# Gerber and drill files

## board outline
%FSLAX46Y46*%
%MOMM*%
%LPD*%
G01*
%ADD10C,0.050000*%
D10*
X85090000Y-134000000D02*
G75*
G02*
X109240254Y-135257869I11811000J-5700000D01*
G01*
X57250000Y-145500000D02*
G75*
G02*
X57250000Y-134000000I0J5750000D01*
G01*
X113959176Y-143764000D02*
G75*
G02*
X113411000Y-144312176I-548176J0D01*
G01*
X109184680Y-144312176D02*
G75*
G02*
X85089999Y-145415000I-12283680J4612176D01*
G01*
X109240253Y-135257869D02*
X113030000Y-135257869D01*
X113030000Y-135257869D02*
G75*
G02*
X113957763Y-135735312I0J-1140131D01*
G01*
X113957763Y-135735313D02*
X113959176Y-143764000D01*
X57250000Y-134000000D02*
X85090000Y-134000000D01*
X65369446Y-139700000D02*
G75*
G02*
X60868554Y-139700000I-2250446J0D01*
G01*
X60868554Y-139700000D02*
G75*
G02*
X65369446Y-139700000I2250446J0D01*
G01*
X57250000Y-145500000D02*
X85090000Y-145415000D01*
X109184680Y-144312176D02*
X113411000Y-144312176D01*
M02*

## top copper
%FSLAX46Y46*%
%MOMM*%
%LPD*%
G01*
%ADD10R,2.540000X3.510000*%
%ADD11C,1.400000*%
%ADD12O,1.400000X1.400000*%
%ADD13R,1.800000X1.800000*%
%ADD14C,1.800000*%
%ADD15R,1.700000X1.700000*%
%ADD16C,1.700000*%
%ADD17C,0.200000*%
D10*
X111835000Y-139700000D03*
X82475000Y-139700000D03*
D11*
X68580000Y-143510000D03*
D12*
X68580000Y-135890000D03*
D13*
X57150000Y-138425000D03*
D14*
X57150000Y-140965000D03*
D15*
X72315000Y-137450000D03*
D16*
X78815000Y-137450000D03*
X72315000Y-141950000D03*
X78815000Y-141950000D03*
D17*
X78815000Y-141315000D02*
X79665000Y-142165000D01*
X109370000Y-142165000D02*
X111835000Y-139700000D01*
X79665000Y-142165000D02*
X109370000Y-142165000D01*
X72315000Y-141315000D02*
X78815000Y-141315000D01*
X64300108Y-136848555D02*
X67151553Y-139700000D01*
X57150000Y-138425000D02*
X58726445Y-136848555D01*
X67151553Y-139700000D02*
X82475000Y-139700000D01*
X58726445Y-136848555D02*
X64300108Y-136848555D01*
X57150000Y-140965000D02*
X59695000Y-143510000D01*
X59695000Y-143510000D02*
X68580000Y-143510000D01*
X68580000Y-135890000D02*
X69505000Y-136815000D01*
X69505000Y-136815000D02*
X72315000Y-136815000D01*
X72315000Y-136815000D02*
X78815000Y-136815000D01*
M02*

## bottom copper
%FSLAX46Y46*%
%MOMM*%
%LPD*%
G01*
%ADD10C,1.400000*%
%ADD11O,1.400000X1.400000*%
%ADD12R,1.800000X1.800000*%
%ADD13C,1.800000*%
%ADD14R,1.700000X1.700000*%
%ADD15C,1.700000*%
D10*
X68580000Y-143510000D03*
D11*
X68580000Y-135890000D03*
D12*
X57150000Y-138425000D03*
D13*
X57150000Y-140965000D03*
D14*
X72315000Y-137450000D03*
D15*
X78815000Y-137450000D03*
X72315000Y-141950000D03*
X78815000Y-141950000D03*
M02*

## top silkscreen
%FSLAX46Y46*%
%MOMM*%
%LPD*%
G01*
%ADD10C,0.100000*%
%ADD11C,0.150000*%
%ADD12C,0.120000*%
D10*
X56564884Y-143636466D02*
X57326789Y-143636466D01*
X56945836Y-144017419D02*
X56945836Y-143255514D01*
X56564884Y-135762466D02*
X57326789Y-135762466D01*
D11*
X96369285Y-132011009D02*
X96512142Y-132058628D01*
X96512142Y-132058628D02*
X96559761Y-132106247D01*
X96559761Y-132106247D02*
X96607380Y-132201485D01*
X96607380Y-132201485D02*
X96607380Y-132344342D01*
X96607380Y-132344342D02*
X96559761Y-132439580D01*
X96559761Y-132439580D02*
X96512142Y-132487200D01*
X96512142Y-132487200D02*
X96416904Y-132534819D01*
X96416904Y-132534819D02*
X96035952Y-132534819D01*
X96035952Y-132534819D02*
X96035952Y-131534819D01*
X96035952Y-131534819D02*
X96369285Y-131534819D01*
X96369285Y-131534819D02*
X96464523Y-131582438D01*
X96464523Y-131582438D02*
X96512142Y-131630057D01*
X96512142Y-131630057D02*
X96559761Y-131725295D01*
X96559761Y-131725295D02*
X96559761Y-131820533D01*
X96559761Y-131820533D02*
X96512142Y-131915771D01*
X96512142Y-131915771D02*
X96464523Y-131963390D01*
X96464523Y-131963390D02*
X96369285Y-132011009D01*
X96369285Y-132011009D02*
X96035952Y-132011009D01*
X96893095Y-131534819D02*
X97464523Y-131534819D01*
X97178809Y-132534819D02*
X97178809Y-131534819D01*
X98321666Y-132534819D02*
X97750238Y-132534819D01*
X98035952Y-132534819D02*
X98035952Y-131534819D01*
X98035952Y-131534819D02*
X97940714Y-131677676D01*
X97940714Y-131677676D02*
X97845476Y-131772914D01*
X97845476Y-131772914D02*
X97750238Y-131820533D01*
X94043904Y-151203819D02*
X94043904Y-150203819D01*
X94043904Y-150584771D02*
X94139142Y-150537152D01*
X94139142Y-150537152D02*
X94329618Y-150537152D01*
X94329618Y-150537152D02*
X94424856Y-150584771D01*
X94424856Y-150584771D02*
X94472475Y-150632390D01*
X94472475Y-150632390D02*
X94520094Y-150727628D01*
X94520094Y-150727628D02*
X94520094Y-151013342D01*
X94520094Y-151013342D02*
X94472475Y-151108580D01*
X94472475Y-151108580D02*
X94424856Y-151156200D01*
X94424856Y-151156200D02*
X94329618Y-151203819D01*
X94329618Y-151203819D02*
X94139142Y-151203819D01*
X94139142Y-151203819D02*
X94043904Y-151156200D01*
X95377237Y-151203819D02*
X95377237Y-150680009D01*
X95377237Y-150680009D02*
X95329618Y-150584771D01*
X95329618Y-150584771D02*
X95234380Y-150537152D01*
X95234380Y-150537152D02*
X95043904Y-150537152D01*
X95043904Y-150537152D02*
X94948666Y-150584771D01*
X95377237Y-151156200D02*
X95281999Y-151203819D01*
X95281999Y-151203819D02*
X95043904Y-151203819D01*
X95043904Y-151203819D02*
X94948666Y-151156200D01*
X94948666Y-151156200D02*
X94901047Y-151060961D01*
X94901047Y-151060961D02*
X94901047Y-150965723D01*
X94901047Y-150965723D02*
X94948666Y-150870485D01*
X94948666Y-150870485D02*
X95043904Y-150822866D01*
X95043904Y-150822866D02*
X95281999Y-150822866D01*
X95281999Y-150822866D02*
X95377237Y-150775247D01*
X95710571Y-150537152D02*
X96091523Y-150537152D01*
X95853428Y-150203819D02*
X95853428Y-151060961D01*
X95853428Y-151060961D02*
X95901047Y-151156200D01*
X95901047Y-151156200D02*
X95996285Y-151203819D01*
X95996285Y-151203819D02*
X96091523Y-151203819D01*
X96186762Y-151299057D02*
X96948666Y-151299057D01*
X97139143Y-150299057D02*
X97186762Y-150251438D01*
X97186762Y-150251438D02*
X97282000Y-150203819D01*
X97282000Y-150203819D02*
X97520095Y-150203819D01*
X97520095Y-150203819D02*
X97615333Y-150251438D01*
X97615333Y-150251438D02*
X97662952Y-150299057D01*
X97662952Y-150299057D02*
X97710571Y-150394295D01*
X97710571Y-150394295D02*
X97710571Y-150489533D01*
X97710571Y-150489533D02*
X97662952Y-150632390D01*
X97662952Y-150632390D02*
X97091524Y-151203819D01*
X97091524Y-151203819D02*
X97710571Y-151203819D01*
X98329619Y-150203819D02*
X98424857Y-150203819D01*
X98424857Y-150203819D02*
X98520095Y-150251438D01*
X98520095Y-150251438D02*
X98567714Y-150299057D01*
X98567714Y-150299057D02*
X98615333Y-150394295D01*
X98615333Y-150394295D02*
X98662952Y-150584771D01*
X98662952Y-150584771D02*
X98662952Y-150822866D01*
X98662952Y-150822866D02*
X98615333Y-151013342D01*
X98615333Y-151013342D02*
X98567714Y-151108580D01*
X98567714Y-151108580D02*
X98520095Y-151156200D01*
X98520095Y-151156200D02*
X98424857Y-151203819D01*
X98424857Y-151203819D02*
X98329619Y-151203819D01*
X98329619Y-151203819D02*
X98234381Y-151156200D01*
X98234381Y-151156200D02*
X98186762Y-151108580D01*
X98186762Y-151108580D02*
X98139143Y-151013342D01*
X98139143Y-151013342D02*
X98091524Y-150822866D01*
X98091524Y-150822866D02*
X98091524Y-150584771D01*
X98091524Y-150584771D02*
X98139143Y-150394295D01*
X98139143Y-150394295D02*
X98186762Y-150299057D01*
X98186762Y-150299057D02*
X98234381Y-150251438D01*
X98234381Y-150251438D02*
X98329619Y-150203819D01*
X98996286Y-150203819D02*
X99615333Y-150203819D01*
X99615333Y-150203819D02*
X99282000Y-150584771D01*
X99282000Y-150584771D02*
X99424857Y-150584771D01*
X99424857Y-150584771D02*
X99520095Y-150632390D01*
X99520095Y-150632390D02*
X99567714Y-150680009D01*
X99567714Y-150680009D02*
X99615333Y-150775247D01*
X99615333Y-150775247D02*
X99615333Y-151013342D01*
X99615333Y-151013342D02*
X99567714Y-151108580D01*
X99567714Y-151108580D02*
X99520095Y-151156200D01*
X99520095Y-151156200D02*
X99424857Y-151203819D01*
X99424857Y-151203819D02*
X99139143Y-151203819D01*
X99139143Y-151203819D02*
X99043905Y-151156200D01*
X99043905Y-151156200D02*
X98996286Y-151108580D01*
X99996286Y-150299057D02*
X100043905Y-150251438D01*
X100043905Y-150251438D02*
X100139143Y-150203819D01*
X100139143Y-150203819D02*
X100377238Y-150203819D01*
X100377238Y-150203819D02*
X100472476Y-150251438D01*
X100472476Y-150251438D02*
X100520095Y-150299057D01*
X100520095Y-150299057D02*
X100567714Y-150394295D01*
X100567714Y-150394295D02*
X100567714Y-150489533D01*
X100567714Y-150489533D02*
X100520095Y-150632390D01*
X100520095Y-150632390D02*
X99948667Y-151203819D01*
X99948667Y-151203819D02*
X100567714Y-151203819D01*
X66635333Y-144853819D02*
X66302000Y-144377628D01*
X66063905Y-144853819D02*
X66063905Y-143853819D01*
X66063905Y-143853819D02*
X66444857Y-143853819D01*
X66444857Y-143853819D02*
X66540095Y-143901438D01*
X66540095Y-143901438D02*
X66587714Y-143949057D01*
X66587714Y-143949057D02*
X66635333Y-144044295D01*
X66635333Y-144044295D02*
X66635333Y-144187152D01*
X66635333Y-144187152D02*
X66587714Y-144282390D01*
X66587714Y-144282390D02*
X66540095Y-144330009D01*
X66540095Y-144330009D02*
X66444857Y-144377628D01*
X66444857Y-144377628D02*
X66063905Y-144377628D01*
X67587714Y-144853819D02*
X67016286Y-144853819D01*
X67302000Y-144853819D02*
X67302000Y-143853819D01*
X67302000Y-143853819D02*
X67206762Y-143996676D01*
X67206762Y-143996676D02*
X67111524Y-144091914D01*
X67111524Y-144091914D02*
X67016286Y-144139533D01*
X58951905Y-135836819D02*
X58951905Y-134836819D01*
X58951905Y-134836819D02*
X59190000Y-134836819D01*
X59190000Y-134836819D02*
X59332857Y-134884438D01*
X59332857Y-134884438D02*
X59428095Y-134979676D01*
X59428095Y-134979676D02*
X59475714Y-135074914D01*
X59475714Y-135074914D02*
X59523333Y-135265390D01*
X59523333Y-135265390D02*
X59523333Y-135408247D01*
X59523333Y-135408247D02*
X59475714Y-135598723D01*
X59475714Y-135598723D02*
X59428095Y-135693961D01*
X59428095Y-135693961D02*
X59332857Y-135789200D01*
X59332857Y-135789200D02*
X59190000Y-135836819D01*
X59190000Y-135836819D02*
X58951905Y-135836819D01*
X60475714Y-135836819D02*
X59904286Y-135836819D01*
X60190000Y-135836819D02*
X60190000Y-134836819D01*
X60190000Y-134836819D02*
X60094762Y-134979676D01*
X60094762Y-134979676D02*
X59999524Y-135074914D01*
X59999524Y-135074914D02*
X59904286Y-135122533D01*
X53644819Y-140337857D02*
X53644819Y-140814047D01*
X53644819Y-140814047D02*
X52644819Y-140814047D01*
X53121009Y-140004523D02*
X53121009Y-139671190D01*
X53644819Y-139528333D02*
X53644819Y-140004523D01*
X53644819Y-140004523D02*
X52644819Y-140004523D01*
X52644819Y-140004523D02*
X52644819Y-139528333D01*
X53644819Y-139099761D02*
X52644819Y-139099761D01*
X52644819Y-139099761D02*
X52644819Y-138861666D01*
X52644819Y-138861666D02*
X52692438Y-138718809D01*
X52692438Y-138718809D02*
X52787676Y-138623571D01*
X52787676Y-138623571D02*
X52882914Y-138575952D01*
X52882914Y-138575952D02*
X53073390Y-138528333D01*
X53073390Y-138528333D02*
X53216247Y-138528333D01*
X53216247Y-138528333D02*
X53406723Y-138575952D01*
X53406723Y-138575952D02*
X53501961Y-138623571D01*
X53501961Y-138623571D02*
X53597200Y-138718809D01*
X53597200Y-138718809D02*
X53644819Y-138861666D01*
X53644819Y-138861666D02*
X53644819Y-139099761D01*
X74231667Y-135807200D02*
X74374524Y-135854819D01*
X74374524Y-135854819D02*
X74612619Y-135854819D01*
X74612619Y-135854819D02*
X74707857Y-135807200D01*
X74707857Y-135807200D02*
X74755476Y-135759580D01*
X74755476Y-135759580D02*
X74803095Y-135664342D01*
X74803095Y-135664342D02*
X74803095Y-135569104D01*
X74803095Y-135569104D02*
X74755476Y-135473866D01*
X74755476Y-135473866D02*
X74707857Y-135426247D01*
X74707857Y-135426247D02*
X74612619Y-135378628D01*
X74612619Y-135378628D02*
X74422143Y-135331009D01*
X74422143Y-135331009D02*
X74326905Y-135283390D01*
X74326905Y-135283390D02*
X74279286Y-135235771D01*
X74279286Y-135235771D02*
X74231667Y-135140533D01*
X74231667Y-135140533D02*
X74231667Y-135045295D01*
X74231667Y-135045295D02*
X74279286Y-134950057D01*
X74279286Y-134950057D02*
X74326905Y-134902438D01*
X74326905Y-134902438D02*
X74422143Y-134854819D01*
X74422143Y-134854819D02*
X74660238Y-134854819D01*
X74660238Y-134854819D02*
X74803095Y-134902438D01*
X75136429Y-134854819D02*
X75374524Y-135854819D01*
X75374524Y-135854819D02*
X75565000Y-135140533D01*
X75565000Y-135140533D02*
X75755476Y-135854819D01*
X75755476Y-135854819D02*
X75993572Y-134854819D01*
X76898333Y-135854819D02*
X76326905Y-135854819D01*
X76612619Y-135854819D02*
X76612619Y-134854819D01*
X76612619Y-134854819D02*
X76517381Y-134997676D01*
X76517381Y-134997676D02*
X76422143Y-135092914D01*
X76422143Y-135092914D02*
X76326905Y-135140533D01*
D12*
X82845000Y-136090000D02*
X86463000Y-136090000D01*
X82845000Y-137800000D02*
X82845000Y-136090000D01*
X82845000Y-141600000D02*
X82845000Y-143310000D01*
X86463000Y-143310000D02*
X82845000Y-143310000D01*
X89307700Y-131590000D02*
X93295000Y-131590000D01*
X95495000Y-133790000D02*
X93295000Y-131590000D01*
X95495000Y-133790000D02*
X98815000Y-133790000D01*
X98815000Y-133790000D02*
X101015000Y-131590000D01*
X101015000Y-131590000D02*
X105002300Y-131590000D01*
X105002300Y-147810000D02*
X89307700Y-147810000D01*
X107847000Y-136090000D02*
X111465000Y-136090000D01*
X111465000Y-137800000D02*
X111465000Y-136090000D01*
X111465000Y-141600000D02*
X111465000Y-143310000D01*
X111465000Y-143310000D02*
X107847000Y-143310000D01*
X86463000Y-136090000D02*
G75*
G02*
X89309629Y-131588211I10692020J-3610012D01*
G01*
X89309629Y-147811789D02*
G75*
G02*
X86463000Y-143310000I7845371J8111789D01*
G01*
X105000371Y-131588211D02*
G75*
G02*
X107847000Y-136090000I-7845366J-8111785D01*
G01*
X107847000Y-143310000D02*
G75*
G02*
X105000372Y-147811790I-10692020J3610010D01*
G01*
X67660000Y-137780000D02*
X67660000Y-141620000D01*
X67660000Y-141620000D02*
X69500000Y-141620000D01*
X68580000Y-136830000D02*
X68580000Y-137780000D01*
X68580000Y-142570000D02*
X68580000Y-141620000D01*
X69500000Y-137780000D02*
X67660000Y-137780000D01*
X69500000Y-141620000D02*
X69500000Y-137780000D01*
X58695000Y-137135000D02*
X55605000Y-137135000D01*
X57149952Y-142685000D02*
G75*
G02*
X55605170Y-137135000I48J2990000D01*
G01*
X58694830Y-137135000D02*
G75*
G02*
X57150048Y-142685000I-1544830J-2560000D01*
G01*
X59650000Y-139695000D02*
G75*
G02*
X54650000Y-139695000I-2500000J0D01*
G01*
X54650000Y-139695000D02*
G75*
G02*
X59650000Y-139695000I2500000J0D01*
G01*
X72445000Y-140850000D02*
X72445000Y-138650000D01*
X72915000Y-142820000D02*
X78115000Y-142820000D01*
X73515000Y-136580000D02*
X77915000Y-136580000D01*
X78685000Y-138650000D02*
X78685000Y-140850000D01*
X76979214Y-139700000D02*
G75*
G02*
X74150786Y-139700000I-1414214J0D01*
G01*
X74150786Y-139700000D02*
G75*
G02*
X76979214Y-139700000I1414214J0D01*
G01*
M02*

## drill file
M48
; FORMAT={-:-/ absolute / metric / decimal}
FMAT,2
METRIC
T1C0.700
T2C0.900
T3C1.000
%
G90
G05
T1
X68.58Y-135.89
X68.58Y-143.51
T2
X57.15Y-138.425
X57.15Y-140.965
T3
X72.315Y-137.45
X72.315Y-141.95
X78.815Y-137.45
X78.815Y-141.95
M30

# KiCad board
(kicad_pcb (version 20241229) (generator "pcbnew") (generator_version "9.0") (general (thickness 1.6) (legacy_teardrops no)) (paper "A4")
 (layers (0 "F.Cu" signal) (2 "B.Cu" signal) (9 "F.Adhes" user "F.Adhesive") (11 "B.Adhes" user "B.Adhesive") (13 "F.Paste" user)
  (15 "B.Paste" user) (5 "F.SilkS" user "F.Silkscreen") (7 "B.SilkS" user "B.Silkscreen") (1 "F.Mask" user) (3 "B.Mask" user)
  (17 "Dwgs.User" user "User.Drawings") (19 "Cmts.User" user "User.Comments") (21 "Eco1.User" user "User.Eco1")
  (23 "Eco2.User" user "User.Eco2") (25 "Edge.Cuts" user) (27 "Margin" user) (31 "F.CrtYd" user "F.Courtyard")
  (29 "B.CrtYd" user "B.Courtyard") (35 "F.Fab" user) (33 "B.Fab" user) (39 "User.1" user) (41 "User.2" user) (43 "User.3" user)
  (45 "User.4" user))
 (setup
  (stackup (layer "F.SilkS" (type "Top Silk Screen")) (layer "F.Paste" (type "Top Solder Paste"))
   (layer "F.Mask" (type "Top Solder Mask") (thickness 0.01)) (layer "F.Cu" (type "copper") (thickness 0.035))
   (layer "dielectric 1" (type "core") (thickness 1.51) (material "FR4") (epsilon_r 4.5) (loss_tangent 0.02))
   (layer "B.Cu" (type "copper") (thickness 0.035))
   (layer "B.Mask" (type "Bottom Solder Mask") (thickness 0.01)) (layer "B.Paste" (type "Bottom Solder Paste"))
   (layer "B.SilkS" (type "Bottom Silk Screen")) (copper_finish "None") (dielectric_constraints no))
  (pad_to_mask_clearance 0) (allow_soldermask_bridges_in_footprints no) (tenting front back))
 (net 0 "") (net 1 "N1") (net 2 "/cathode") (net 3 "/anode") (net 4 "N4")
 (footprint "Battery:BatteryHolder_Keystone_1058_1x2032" (layer "F.Cu") (at 97.155 139.7 180)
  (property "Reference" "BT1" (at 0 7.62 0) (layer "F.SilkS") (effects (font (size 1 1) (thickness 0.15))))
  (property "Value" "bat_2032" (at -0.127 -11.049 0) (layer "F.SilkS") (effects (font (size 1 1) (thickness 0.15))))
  (fp_line (start 14.31 3.61) (end 10.692 3.61) (stroke (width 0.12) (type solid)) (layer "F.SilkS"))
  (fp_line (start 14.31 1.9) (end 14.31 3.61) (stroke (width 0.12) (type solid)) (layer "F.SilkS"))
  (fp_line (start 14.31 -1.9) (end 14.31 -3.61) (stroke (width 0.12) (type solid)) (layer "F.SilkS"))
  (fp_line (start 10.692 -3.61) (end 14.31 -3.61) (stroke (width 0.12) (type solid)) (layer "F.SilkS"))
  (fp_line (start 7.8473 8.11) (end 3.86 8.11) (stroke (width 0.12) (type solid)) (layer "F.SilkS"))
  (fp_line (start 1.66 5.91) (end 3.86 8.11) (stroke (width 0.12) (type solid)) (layer "F.SilkS"))
  (fp_line (start 1.66 5.91) (end -1.66 5.91) (stroke (width 0.12) (type solid)) (layer "F.SilkS"))
  (fp_line (start -1.66 5.91) (end -3.86 8.11) (stroke (width 0.12) (type solid)) (layer "F.SilkS"))
  (fp_line (start -3.86 8.11) (end -7.8473 8.11) (stroke (width 0.12) (type solid)) (layer "F.SilkS"))
  (fp_line (start -7.8473 -8.11) (end 7.8473 -8.11) (stroke (width 0.12) (type solid)) (layer "F.SilkS"))
  (fp_line (start -10.692 3.61) (end -14.31 3.61) (stroke (width 0.12) (type solid)) (layer "F.SilkS"))
  (fp_line (start -14.31 1.9) (end -14.31 3.61) (stroke (width 0.12) (type solid)) (layer "F.SilkS"))
  (fp_line (start -14.31 -1.9) (end -14.31 -3.61) (stroke (width 0.12) (type solid)) (layer "F.SilkS"))
  (fp_line (start -14.31 -3.61) (end -10.692 -3.61) (stroke (width 0.12) (type solid)) (layer "F.SilkS"))
  (fp_arc (start 10.692 3.61) (mid 9.538084 6.031244) (end 7.845371 8.111789) (stroke (width 0.12) (type solid)) (layer "F.SilkS"))
  (fp_arc (start 7.845371 -8.111789) (mid 9.538085 -6.031244) (end 10.692 -3.61) (stroke (width 0.12) (type solid)) (layer "F.SilkS"))
  (fp_arc (start -7.845371 8.111789) (mid -9.538085 6.031244) (end -10.692 3.61) (stroke (width 0.12) (type solid)) (layer "F.SilkS"))
  (fp_arc (start -10.692 -3.61) (mid -9.538084 -6.031244) (end -7.845371 -8.111789) (stroke (width 0.12) (type solid)) (layer "F.SilkS"))
  (pad "1" smd rect (at -14.68 0 180) (size 2.54 3.51) (layers "F.Cu" "F.Mask" "F.Paste") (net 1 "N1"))
  (pad "2" smd rect (at 14.68 0 180) (size 2.54 3.51) (layers "F.Cu" "F.Mask" "F.Paste") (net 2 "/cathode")))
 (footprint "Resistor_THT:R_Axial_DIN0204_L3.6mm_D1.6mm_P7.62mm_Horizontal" (layer "F.Cu") (at 68.58 143.51 90)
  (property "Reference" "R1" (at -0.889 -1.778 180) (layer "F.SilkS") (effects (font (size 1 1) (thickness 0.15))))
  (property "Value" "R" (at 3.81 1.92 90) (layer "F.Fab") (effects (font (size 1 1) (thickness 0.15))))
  (fp_line (start 5.73 -0.92) (end 1.89 -0.92) (stroke (width 0.12) (type solid)) (layer "F.SilkS"))
  (fp_line (start 1.89 -0.92) (end 1.89 0.92) (stroke (width 0.12) (type solid)) (layer "F.SilkS"))
  (fp_line (start 6.68 0) (end 5.73 0) (stroke (width 0.12) (type solid)) (layer "F.SilkS"))
  (fp_line (start 0.94 0) (end 1.89 0) (stroke (width 0.12) (type solid)) (layer "F.SilkS"))
  (fp_line (start 5.73 0.92) (end 5.73 -0.92) (stroke (width 0.12) (type solid)) (layer "F.SilkS"))
  (fp_line (start 1.89 0.92) (end 5.73 0.92) (stroke (width 0.12) (type solid)) (layer "F.SilkS"))
  (pad "1" thru_hole circle (at 0 0 90) (size 1.4 1.4) (drill 0.7) (layers "*.Cu" "*.Mask") (remove_unused_layers no) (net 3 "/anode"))
  (pad "2" thru_hole oval (at 7.62 0 90) (size 1.4 1.4) (drill 0.7) (layers "*.Cu" "*.Mask") (remove_unused_layers no) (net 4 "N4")))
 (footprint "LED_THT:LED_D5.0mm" (layer "F.Cu") (at 57.15 138.425 -90)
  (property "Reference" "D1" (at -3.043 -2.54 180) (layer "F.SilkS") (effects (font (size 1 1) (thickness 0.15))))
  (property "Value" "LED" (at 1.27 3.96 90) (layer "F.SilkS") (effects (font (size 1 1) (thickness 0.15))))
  (fp_line (start -1.29 -1.545) (end -1.29 1.545) (stroke (width 0.12) (type solid)) (layer "F.SilkS"))
  (fp_arc (start 4.26 0.000048) (mid 2.071756 2.880501) (end -1.29 1.54483) (stroke (width 0.12) (type solid)) (layer "F.SilkS"))
  (fp_arc (start -1.29 -1.54483) (mid 2.071756 -2.880501) (end 4.26 -0.000048) (stroke (width 0.12) (type solid)) (layer "F.SilkS"))
  (fp_circle (center 1.27 0) (end 3.77 0) (stroke (width 0.12) (type solid)) (fill no) (layer "F.SilkS"))
  (pad "1" thru_hole rect (at 0 0 270) (size 1.8 1.8) (drill 0.9) (layers "*.Cu" "*.Mask") (remove_unused_layers no) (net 2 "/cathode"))
  (pad "2" thru_hole circle (at 2.54 0 270) (size 1.8 1.8) (drill 0.9) (layers "*.Cu" "*.Mask") (remove_unused_layers no) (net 3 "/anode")))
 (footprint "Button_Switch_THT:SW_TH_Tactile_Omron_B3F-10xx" (layer "F.Cu") (at 72.315 137.45)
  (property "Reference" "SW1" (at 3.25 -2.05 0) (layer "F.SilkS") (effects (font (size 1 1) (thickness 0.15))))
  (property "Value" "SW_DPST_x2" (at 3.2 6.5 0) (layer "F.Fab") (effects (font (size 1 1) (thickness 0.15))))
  (fp_line (start 0.13 3.4) (end 0.13 1.2) (stroke (width 0.12) (type solid)) (layer "F.SilkS"))
  (fp_line (start 0.6 5.37) (end 5.8 5.37) (stroke (width 0.12) (type solid)) (layer "F.SilkS"))
  (fp_line (start 1.2 -0.87) (end 5.6 -0.87) (stroke (width 0.12) (type solid)) (layer "F.SilkS"))
  (fp_line (start 6.37 1.2) (end 6.37 3.4) (stroke (width 0.12) (type solid)) (layer "F.SilkS"))
  (fp_circle (center 3.25 2.25) (end 4.25 3.25) (stroke (width 0.12) (type solid)) (fill no) (layer "F.SilkS"))
  (pad "1" thru_hole rect (at 0 0) (size 1.7 1.7) (drill 1) (layers "*.Cu" "*.Mask") (remove_unused_layers no) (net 4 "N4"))
  (pad "1" thru_hole circle (at 6.5 0) (size 1.7 1.7) (drill 1) (layers "*.Cu" "*.Mask") (remove_unused_layers no) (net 4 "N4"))
  (pad "2" thru_hole circle (at 0 4.5) (size 1.7 1.7) (drill 1) (layers "*.Cu" "*.Mask") (remove_unused_layers no) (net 1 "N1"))
  (pad "2" thru_hole circle (at 6.5 4.5) (size 1.7 1.7) (drill 1) (layers "*.Cu" "*.Mask") (remove_unused_layers no) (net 1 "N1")))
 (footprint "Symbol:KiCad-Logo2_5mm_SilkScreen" (layer "B.Cu") (at 96.901 136.398 180)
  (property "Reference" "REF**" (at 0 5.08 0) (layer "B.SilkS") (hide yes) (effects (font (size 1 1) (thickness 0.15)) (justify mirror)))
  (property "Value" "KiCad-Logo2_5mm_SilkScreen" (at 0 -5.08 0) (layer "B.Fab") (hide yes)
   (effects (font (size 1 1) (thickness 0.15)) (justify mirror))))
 (gr_arc (start 85.09 134) (mid 97.583145 126.603268) (end 109.240254 135.257869) (stroke (width 0.05) (type default)) (locked yes)
  (layer "Edge.Cuts"))
 (gr_arc (start 57.25 145.5) (mid 51.5 139.75) (end 57.25 134) (stroke (width 0.05) (type default)) (locked yes) (layer "Edge.Cuts"))
 (gr_arc (start 113.959176 143.764) (mid 113.798619 144.151619) (end 113.411 144.312176) (stroke (width 0.05) (type default)) (locked yes)
  (layer "Edge.Cuts"))
 (gr_arc (start 109.18468 144.312176) (mid 97.500927 152.80729) (end 85.09 145.415) (stroke (width 0.05) (type default)) (locked yes)
  (layer "Edge.Cuts"))
 (gr_line (start 109.240253 135.257869) (end 113.03 135.257869) (stroke (width 0.05) (type default)) (locked yes) (layer "Edge.Cuts"))
 (gr_arc (start 113.03 135.257869) (mid 113.551703 135.384232) (end 113.957763 135.735312) (stroke (width 0.05) (type default)) (locked yes)
  (layer "Edge.Cuts"))
 (gr_line (start 113.957763 135.735313) (end 113.959176 143.764) (stroke (width 0.05) (type default)) (locked yes) (layer "Edge.Cuts"))
 (gr_line (start 57.25 134) (end 85.09 134) (stroke (width 0.05) (type default)) (locked yes) (layer "Edge.Cuts"))
 (gr_circle (center 63.119 139.7) (end 63.754 141.859) (stroke (width 0.05) (type default)) (fill no) (layer "Edge.Cuts"))
 (gr_line (start 57.25 145.5) (end 85.09 145.415) (stroke (width 0.05) (type default)) (locked yes) (layer "Edge.Cuts"))
 (gr_line (start 109.18468 144.312176) (end 113.411 144.312176) (stroke (width 0.05) (type default)) (locked yes) (layer "Edge.Cuts"))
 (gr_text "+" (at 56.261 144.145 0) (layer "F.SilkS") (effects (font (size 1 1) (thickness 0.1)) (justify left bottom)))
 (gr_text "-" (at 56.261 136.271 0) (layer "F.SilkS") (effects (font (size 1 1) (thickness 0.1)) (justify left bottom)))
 (segment (start 78.815 141.315) (end 79.665 142.165) (width 0.2) (layer "F.Cu") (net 1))
 (segment (start 109.37 142.165) (end 111.835 139.7) (width 0.2) (layer "F.Cu") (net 1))
 (segment (start 79.665 142.165) (end 109.37 142.165) (width 0.2) (layer "F.Cu") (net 1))
 (segment (start 72.315 141.315) (end 78.815 141.315) (width 0.2) (layer "F.Cu") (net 1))
 (segment (start 64.300108 136.848555) (end 67.151553 139.7) (width 0.2) (layer "F.Cu") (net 2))
 (segment (start 57.15 138.425) (end 58.726445 136.848555) (width 0.2) (layer "F.Cu") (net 2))
 (segment (start 67.151553 139.7) (end 82.475 139.7) (width 0.2) (layer "F.Cu") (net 2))
 (segment (start 58.726445 136.848555) (end 64.300108 136.848555) (width 0.2) (layer "F.Cu") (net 2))
 (segment (start 57.15 140.965) (end 59.695 143.51) (width 0.2) (layer "F.Cu") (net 3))
 (segment (start 59.695 143.51) (end 68.58 143.51) (width 0.2) (layer "F.Cu") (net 3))
 (segment (start 68.58 135.89) (end 69.505 136.815) (width 0.2) (layer "F.Cu") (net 4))
 (segment (start 69.505 136.815) (end 72.315 136.815) (width 0.2) (layer "F.Cu") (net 4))
 (segment (start 72.315 136.815) (end 78.815 136.815) (width 0.2) (layer "F.Cu") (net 4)))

